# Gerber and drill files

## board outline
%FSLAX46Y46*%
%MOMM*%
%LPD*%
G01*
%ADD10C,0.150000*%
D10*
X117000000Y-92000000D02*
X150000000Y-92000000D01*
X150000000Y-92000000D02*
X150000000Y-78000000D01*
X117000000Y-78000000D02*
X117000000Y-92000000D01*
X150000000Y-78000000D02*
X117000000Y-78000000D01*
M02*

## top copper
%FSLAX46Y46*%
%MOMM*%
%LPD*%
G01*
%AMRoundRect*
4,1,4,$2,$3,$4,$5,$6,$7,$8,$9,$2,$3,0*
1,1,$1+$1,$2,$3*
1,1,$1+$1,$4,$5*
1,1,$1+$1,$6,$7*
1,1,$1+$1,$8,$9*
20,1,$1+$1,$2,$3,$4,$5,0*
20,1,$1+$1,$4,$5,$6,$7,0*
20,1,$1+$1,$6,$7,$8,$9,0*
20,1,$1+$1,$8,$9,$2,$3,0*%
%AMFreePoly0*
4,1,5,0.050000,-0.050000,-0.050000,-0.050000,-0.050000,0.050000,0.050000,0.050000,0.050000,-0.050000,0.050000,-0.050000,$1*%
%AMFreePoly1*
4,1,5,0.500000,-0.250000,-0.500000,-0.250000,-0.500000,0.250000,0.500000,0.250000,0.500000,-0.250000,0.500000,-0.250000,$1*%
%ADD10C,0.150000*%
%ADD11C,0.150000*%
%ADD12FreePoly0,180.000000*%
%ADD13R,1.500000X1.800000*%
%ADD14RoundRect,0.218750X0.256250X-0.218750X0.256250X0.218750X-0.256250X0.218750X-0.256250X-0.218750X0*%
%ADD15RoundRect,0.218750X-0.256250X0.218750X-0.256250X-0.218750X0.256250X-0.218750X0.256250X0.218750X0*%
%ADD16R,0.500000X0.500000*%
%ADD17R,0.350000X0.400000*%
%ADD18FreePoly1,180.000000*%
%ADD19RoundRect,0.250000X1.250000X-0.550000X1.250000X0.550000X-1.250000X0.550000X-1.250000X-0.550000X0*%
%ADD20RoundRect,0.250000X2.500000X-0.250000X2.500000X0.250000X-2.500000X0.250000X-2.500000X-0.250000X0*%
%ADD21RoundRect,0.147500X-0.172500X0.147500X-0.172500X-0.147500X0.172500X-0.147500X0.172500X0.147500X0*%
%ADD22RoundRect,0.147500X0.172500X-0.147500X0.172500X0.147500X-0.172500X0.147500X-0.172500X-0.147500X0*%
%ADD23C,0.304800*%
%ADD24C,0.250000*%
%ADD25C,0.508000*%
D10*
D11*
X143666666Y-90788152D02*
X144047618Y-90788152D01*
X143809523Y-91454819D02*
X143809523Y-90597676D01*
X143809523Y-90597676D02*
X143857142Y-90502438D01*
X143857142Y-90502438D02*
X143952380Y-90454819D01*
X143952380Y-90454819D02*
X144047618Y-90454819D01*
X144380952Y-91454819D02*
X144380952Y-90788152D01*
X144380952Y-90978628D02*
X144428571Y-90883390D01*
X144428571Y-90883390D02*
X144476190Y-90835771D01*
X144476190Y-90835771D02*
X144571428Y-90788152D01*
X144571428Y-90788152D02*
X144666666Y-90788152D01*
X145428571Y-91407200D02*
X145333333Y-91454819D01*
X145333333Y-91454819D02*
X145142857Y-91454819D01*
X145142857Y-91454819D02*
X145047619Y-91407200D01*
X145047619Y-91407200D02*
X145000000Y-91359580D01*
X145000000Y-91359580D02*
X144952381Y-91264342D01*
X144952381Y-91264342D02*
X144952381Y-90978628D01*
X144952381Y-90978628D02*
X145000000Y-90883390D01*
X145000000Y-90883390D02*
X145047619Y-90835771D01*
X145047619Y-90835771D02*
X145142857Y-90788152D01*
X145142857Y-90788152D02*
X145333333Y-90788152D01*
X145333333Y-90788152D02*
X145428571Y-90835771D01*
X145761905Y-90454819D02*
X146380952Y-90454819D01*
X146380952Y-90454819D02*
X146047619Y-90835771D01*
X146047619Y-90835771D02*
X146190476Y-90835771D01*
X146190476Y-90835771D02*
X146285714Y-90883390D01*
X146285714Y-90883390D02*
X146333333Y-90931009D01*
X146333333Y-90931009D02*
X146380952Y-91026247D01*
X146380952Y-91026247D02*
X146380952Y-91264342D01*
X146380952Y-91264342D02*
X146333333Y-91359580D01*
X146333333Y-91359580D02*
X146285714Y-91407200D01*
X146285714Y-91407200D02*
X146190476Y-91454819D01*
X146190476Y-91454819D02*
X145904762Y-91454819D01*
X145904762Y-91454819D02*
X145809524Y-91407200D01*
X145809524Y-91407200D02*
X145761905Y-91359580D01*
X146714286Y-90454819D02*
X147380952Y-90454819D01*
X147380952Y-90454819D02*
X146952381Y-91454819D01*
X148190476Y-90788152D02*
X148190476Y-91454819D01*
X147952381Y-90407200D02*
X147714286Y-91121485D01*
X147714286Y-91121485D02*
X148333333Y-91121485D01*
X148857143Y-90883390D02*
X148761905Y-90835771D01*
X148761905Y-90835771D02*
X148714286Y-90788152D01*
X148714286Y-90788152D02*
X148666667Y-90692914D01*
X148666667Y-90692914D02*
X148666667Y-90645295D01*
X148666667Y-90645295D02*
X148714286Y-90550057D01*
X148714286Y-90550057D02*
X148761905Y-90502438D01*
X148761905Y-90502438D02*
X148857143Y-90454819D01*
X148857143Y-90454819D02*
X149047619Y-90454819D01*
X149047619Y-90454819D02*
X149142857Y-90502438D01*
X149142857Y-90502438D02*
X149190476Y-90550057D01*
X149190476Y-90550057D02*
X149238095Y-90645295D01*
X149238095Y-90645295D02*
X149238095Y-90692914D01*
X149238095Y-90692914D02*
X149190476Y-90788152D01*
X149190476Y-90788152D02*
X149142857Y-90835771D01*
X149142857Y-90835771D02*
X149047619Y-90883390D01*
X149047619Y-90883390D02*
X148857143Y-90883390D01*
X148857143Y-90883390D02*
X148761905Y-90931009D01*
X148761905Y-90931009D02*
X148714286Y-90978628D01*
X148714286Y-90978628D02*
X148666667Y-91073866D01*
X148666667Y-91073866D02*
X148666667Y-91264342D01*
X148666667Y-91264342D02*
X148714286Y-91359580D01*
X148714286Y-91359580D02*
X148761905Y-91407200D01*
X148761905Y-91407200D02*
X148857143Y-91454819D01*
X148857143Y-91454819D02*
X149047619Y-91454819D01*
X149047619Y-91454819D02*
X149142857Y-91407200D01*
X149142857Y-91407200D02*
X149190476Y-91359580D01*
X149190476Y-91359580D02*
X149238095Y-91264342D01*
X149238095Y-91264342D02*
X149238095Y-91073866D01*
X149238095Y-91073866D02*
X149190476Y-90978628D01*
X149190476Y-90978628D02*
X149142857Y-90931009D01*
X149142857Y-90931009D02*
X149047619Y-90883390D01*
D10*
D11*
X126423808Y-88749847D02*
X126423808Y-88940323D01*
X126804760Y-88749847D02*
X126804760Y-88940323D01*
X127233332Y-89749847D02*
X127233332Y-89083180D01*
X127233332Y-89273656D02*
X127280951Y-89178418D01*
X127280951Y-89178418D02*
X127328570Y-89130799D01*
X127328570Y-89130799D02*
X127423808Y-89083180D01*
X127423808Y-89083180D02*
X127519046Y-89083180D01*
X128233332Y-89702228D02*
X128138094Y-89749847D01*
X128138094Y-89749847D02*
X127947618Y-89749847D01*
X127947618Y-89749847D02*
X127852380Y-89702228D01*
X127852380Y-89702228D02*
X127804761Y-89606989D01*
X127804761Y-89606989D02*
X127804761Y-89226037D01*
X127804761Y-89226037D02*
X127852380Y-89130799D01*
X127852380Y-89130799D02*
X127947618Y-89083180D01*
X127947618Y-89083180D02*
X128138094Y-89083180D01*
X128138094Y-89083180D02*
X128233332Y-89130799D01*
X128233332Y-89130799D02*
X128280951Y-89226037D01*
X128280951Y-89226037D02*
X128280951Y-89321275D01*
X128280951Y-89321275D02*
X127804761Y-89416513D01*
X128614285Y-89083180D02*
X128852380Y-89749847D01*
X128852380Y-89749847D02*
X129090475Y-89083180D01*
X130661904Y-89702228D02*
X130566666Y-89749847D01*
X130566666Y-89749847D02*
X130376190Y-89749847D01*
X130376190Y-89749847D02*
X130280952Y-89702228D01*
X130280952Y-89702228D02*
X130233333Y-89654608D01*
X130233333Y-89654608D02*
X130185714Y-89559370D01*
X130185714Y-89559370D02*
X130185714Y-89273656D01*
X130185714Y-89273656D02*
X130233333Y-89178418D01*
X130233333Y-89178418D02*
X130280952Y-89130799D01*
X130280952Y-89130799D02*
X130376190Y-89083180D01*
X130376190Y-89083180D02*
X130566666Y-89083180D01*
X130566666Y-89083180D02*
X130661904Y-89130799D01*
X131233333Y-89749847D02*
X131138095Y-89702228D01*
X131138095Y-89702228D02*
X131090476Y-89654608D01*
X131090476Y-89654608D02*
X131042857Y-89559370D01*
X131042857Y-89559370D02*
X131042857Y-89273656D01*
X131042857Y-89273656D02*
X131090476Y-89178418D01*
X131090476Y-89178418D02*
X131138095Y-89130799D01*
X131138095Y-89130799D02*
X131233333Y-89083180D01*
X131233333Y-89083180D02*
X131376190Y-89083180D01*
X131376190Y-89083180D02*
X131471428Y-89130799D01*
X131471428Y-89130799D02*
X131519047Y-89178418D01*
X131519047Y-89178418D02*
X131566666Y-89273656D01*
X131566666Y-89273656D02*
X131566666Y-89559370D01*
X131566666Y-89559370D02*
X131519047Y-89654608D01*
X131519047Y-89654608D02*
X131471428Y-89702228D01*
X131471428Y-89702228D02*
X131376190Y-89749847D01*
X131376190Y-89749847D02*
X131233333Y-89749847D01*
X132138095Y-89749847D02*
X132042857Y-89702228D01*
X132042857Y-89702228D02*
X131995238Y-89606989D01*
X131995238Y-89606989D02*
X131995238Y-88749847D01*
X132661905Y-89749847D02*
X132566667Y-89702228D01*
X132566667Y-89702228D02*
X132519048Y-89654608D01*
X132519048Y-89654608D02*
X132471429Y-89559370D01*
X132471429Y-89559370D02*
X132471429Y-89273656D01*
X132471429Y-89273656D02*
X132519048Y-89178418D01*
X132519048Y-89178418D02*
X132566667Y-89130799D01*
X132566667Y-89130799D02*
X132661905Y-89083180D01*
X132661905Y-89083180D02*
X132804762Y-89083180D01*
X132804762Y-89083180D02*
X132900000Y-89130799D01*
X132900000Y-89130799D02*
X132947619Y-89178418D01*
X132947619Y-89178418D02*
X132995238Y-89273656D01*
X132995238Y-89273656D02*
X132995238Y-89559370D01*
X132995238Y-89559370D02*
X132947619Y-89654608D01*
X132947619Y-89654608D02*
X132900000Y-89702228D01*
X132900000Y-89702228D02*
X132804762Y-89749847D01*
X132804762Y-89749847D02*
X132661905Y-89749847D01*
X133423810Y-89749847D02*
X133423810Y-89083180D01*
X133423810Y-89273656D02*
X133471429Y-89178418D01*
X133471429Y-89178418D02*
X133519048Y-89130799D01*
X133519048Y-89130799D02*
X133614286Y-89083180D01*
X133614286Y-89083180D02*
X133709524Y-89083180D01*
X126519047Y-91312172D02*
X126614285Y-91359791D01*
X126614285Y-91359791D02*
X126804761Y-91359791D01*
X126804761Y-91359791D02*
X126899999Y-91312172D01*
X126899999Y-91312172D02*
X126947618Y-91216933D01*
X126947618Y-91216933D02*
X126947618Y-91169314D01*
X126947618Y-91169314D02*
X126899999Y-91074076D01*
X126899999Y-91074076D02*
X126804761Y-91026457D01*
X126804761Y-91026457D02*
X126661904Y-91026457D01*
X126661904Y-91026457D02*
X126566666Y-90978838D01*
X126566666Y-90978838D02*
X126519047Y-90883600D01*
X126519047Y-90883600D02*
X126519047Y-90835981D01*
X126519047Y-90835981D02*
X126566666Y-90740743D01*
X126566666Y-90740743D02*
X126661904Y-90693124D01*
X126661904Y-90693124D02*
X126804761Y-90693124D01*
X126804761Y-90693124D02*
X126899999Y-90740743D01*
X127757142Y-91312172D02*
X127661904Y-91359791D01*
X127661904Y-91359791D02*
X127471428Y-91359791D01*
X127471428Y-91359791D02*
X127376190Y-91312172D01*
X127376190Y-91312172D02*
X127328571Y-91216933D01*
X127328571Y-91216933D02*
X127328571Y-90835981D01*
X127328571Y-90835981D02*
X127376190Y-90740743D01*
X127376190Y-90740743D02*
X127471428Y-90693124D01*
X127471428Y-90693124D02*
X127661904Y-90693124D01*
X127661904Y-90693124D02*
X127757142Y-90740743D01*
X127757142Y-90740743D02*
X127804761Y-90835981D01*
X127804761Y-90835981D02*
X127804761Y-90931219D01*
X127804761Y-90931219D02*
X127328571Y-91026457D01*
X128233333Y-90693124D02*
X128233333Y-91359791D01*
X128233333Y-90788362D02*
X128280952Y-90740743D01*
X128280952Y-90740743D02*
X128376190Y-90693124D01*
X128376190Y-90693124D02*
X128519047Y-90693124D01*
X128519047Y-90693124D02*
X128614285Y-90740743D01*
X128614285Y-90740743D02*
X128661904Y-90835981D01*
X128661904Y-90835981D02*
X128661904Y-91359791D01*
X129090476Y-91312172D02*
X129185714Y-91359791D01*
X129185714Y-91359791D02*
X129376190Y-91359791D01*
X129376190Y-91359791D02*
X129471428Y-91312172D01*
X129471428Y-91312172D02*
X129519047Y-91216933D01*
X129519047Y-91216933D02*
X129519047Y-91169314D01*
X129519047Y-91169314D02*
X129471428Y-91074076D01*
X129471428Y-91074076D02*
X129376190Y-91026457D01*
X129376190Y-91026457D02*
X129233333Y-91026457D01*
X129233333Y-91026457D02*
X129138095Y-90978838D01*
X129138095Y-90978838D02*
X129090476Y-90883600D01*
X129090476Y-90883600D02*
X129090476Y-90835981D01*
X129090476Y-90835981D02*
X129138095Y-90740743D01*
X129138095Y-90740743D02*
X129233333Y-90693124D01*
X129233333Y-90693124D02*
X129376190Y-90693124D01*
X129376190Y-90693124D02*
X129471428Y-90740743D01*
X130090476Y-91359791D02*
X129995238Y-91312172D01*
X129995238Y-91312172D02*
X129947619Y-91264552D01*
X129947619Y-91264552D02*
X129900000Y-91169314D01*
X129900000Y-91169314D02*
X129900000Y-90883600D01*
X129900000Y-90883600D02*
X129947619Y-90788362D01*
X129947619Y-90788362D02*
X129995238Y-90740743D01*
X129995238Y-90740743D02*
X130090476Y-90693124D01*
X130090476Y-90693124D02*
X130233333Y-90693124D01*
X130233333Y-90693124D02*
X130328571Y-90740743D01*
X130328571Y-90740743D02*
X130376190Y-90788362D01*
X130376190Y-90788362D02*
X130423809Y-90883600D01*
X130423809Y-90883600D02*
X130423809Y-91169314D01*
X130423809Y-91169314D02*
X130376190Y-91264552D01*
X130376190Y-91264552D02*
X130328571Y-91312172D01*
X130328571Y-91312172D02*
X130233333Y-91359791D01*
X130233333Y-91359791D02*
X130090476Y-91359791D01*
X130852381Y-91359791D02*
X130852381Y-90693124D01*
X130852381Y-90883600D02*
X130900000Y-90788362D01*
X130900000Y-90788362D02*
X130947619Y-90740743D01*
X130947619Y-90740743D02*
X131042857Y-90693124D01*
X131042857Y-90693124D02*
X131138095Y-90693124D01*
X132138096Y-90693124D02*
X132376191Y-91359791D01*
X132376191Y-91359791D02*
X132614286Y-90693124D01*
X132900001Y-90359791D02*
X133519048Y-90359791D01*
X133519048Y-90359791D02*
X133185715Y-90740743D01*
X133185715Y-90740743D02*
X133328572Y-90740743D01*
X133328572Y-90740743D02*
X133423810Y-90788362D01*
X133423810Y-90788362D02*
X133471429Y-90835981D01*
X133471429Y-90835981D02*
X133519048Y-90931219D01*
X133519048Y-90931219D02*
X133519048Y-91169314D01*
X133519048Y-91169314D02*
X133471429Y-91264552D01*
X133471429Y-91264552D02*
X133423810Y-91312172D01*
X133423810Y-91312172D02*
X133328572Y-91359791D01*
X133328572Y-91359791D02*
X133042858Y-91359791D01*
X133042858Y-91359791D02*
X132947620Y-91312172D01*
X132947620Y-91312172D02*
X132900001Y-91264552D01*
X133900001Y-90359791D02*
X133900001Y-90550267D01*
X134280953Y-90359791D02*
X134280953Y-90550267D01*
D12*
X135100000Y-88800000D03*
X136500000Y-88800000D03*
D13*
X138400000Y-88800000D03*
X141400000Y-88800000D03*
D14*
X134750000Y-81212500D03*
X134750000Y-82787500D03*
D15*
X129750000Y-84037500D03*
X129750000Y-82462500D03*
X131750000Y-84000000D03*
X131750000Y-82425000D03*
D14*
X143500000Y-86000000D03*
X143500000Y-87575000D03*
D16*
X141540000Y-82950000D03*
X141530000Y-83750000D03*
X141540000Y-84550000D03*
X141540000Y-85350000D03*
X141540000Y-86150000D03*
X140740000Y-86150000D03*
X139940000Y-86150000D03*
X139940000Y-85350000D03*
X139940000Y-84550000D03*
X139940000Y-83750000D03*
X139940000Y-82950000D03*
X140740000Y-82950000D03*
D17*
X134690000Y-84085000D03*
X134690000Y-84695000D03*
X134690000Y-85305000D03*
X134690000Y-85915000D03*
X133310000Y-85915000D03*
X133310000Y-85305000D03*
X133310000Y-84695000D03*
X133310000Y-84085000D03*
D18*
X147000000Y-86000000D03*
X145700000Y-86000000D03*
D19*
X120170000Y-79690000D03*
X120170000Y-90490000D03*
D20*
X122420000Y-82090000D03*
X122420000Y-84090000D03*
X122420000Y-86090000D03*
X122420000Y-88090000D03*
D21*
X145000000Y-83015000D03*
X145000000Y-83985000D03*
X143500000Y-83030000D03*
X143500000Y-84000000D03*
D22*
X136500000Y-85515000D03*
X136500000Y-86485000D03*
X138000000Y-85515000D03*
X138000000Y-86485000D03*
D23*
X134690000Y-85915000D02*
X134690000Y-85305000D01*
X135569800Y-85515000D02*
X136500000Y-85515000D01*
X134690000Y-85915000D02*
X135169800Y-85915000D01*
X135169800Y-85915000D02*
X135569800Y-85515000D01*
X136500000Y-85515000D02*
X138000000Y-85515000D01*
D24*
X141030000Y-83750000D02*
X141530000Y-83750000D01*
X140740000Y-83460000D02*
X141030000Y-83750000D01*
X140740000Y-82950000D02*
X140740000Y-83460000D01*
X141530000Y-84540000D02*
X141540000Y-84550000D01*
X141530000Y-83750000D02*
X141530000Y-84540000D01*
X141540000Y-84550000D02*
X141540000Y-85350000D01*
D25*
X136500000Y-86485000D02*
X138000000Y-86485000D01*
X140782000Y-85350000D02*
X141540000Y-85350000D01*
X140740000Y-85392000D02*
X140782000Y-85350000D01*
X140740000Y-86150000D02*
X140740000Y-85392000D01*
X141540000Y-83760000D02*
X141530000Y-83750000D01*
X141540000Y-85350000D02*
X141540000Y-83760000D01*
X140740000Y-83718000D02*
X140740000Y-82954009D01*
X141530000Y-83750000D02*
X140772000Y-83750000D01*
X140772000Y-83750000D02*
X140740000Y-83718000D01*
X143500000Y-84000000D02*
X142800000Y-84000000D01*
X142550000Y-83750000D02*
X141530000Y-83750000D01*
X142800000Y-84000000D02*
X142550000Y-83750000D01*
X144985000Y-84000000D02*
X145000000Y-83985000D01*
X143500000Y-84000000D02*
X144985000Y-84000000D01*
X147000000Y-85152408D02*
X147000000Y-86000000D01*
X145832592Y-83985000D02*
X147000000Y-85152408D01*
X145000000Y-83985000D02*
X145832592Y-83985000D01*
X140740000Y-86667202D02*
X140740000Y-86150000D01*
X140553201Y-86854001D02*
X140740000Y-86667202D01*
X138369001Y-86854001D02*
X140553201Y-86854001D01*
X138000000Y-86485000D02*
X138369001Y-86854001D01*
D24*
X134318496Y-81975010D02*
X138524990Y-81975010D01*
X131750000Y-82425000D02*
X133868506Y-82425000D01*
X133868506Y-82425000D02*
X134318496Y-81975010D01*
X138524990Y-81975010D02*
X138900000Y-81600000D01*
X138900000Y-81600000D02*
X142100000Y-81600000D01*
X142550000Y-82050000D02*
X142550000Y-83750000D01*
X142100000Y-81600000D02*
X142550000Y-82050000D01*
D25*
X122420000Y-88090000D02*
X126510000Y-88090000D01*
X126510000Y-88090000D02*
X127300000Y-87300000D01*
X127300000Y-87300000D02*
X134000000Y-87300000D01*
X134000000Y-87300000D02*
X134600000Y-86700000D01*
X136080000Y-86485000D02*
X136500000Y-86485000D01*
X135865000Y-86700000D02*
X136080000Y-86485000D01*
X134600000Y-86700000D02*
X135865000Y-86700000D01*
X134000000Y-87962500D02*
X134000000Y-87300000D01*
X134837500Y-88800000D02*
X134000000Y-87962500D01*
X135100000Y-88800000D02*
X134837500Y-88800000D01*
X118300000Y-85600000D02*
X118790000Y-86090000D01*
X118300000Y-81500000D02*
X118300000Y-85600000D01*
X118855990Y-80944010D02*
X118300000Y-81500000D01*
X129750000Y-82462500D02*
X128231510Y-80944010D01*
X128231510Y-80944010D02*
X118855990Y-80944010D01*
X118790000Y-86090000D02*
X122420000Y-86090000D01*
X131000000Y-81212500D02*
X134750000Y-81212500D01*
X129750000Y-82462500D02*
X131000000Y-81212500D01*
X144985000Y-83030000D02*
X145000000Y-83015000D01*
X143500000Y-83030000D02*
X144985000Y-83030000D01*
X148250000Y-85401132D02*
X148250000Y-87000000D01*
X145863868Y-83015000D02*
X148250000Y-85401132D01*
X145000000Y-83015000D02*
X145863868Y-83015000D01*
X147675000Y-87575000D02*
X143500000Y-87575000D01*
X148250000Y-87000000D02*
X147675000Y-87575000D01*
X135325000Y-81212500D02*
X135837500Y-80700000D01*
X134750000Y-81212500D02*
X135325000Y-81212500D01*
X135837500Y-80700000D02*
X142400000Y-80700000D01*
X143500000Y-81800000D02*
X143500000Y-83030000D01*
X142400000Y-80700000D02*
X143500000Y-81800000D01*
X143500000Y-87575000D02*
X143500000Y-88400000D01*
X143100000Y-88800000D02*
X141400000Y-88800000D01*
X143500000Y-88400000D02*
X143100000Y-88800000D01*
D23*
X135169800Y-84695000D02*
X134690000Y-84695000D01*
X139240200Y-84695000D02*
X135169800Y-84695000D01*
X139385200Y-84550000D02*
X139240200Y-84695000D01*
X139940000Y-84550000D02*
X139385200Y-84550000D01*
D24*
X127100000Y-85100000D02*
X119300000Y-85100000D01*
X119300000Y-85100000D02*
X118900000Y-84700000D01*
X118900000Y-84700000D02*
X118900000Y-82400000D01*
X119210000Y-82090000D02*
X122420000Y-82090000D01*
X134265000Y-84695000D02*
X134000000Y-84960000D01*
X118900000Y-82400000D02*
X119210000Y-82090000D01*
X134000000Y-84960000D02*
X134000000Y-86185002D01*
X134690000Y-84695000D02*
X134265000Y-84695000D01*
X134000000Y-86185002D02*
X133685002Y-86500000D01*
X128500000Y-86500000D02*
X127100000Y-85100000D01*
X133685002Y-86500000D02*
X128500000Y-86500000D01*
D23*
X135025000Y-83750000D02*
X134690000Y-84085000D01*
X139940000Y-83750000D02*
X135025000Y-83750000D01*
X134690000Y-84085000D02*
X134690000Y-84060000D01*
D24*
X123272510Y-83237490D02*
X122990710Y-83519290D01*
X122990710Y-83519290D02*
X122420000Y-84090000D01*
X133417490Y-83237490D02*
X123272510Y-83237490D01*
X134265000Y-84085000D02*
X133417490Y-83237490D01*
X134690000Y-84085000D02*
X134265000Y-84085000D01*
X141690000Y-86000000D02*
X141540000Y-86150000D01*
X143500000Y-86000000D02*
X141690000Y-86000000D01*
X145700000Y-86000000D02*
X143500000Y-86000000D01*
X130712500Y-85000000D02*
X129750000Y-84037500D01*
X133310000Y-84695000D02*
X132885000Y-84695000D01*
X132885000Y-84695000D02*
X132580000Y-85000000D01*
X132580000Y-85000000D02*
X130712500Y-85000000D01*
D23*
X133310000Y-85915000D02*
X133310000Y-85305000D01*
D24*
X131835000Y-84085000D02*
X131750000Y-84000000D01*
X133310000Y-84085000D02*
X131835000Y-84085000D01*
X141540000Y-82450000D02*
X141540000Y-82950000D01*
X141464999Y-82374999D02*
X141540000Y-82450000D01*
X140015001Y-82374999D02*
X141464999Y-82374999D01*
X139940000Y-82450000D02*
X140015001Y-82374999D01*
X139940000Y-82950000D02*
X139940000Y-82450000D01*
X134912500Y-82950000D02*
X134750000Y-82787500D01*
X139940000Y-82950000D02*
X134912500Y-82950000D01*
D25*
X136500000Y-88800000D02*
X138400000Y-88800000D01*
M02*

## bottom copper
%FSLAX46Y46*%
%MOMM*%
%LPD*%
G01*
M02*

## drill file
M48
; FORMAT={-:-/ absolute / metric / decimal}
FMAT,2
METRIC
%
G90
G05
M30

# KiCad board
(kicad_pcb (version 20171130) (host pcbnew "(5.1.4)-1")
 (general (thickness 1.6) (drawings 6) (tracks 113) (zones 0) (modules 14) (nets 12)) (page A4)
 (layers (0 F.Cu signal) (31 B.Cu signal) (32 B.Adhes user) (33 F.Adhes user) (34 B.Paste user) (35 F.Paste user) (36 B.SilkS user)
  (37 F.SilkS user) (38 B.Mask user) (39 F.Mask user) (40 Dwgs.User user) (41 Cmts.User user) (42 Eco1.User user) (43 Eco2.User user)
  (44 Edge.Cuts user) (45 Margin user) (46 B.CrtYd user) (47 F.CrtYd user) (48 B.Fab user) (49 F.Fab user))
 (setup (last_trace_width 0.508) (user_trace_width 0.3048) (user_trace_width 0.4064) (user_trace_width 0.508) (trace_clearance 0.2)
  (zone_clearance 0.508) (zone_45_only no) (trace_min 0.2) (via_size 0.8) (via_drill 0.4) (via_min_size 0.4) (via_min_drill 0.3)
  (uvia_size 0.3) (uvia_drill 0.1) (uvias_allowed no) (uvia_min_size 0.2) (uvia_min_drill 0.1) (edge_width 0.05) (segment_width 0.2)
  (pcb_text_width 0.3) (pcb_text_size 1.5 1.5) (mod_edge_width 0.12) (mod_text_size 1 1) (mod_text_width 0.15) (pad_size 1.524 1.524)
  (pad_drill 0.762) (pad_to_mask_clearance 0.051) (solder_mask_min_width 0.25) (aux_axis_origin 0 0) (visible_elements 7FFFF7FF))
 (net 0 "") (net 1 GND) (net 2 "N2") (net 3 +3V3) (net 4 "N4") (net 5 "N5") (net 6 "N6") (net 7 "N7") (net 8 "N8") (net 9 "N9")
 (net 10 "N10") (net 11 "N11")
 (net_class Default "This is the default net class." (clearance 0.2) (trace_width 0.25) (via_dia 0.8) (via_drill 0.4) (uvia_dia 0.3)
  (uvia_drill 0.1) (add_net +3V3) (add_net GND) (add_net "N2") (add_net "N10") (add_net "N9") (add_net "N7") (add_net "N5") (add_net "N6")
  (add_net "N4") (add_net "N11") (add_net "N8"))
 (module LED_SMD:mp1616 (layer F.Cu) (at 135.8 88.9 180)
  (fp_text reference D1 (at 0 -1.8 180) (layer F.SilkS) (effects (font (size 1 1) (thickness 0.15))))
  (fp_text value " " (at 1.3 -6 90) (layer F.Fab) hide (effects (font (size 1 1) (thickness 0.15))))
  (pad 1 smd custom (at 0.7 0.1 180) (size 0.1 0.1) (layers F.Cu F.Paste F.Mask) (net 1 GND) (options (clearance outline) (anchor rect))
   (primitives))
  (pad 2 smd custom (at -0.7 0.1 180) (size 0.1 0.1) (layers F.Cu F.Paste F.Mask) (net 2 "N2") (options (clearance outline) (anchor rect))
   (primitives)))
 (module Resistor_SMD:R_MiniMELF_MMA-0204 (layer F.Cu) (at 139.9 88.8 180)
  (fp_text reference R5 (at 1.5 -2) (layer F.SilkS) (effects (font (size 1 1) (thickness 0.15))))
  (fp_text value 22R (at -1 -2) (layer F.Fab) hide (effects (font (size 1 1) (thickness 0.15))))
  (pad 2 smd rect (at 1.5 0 180) (size 1.5 1.8) (layers F.Cu F.Paste F.Mask) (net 2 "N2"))
  (pad 1 smd rect (at -1.5 0 180) (size 1.5 1.8) (layers F.Cu F.Paste F.Mask) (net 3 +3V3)))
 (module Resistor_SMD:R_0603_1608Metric (layer F.Cu) (at 134.75 82 90)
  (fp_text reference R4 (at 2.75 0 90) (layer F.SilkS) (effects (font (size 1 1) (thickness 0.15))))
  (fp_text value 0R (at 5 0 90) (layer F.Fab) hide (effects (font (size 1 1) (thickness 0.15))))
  (pad 2 smd roundrect (at 0.7875 0 90) (size 0.875 0.95) (layers F.Cu F.Paste F.Mask) (roundrect_rratio 0.25) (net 3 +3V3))
  (pad 1 smd roundrect (at -0.7875 0 90) (size 0.875 0.95) (layers F.Cu F.Paste F.Mask) (roundrect_rratio 0.25) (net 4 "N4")))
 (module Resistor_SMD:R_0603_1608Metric (layer F.Cu) (at 129.75 83.25 270)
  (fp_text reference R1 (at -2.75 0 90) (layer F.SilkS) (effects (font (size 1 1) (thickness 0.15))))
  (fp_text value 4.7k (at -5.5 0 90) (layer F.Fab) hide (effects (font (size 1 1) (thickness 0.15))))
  (pad 2 smd roundrect (at 0.7875 0 270) (size 0.875 0.95) (layers F.Cu F.Paste F.Mask) (roundrect_rratio 0.25) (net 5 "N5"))
  (pad 1 smd roundrect (at -0.7875 0 270) (size 0.875 0.95) (layers F.Cu F.Paste F.Mask) (roundrect_rratio 0.25) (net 3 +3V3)))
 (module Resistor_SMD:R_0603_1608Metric (layer F.Cu) (at 131.75 83.2125 270)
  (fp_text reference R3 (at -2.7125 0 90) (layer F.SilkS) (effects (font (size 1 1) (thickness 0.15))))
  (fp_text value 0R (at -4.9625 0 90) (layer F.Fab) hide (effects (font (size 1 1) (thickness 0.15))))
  (pad 2 smd roundrect (at 0.7875 0 270) (size 0.875 0.95) (layers F.Cu F.Paste F.Mask) (roundrect_rratio 0.25) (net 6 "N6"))
  (pad 1 smd roundrect (at -0.7875 0 270) (size 0.875 0.95) (layers F.Cu F.Paste F.Mask) (roundrect_rratio 0.25) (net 1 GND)))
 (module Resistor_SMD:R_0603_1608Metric (layer F.Cu) (at 143.5 86.7875 90)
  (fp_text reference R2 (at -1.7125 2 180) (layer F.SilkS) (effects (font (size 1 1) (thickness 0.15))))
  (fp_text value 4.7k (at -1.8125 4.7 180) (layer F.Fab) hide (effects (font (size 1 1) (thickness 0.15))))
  (pad 2 smd roundrect (at 0.7875 0 90) (size 0.875 0.95) (layers F.Cu F.Paste F.Mask) (roundrect_rratio 0.25) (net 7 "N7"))
  (pad 1 smd roundrect (at -0.7875 0 90) (size 0.875 0.95) (layers F.Cu F.Paste F.Mask) (roundrect_rratio 0.25) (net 3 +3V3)))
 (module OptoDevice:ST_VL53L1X (layer F.Cu) (at 140.74 84.55 270)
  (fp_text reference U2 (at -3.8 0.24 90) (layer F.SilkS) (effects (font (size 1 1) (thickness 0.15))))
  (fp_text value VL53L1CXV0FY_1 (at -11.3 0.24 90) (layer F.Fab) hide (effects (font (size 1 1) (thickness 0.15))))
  (pad 1 smd rect (at -1.6 -0.8) (size 0.5 0.5) (layers F.Cu F.Paste F.Mask) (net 4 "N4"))
  (pad 2 smd rect (at -0.8 -0.79) (size 0.5 0.5) (layers F.Cu F.Paste F.Mask) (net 1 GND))
  (pad 3 smd rect (at 0 -0.8) (size 0.5 0.5) (layers F.Cu F.Paste F.Mask) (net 1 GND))
  (pad 4 smd rect (at 0.8 -0.8) (size 0.5 0.5) (layers F.Cu F.Paste F.Mask) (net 1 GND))
  (pad 5 smd rect (at 1.6 -0.8) (size 0.5 0.5) (layers F.Cu F.Paste F.Mask) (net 7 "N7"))
  (pad 6 smd rect (at 1.6 0) (size 0.5 0.5) (layers F.Cu F.Paste F.Mask) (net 1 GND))
  (pad 7 smd rect (at 1.6 0.8) (size 0.5 0.5) (layers F.Cu F.Paste F.Mask) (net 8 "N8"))
  (pad 8 smd rect (at 0.8 0.8) (size 0.5 0.5) (layers F.Cu F.Paste F.Mask))
  (pad 9 smd rect (at 0 0.8) (size 0.5 0.5) (layers F.Cu F.Paste F.Mask) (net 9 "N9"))
  (pad 10 smd rect (at -0.8 0.8) (size 0.5 0.5) (layers F.Cu F.Paste F.Mask) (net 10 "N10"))
  (pad 11 smd rect (at -1.6 0.8) (size 0.5 0.5) (layers F.Cu F.Paste F.Mask) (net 4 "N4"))
  (pad 12 smd rect (at -1.6 0) (size 0.5 0.5) (layers F.Cu F.Paste F.Mask) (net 1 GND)))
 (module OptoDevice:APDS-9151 (layer F.Cu) (at 134 85)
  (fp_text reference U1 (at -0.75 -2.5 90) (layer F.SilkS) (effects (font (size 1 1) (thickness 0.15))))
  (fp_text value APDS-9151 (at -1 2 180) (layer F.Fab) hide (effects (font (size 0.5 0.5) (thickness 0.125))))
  (pad 8 smd rect (at 0.69 -0.915) (size 0.35 0.4) (layers F.Cu F.Paste F.Mask) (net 10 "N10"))
  (pad 7 smd rect (at 0.69 -0.305) (size 0.35 0.4) (layers F.Cu F.Paste F.Mask) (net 9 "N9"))
  (pad 6 smd rect (at 0.69 0.305 180) (size 0.35 0.4) (layers F.Cu F.Paste F.Mask) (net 3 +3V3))
  (pad 5 smd rect (at 0.69 0.915) (size 0.35 0.4) (layers F.Cu F.Paste F.Mask) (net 3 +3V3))
  (pad 4 smd rect (at -0.69 0.915) (size 0.35 0.4) (layers F.Cu F.Paste F.Mask) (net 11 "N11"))
  (pad 3 smd rect (at -0.69 0.305) (size 0.35 0.4) (layers F.Cu F.Paste F.Mask) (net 11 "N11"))
  (pad 2 smd rect (at -0.69 -0.305) (size 0.35 0.4) (layers F.Cu F.Paste F.Mask) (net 5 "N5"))
  (pad 1 smd rect (at -0.69 -0.915) (size 0.35 0.4) (layers F.Cu F.Paste F.Mask) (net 6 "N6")))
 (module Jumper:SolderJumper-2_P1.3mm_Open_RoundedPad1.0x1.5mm (layer F.Cu) (at 146.35 86 180)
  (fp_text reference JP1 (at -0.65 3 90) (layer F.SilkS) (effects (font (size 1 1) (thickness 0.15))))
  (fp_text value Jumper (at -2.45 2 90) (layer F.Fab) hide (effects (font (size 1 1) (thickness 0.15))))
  (pad 1 smd custom (at -0.65 0 180) (size 1 0.5) (layers F.Cu F.Mask) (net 1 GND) (zone_connect 2)
   (options (clearance outline) (anchor rect)) (primitives))
  (pad 2 smd custom (at 0.65 0 180) (size 1 0.5) (layers F.Cu F.Mask) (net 7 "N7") (zone_connect 2)
   (options (clearance outline) (anchor rect)) (primitives)))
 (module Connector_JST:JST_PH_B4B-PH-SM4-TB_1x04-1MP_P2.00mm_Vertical (layer F.Cu) (at 121.92 85.09 90)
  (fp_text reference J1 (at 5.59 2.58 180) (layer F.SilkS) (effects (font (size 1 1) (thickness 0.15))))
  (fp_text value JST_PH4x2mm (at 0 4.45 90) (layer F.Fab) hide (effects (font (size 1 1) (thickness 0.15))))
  (pad MP smd roundrect (at 5.4 -1.75 90) (size 1.6 3) (layers F.Cu F.Paste F.Mask) (roundrect_rratio 0.15625))
  (pad MP smd roundrect (at -5.4 -1.75 90) (size 1.6 3) (layers F.Cu F.Paste F.Mask) (roundrect_rratio 0.15625))
  (pad 4 smd roundrect (at 3 0.5 90) (size 1 5.5) (layers F.Cu F.Paste F.Mask) (roundrect_rratio 0.25) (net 9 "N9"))
  (pad 3 smd roundrect (at 1 0.5 90) (size 1 5.5) (layers F.Cu F.Paste F.Mask) (roundrect_rratio 0.25) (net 10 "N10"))
  (pad 2 smd roundrect (at -1 0.5 90) (size 1 5.5) (layers F.Cu F.Paste F.Mask) (roundrect_rratio 0.25) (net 3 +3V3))
  (pad 1 smd roundrect (at -3 0.5 90) (size 1 5.5) (layers F.Cu F.Paste F.Mask) (roundrect_rratio 0.25) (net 1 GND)))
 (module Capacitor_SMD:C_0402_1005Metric (layer F.Cu) (at 145 83.5 270)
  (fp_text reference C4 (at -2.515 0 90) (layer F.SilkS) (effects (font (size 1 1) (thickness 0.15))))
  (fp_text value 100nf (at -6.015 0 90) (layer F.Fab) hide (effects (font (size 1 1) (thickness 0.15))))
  (pad 1 smd roundrect (at -0.485 0 270) (size 0.59 0.64) (layers F.Cu F.Paste F.Mask) (roundrect_rratio 0.25) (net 3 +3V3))
  (pad 2 smd roundrect (at 0.485 0 270) (size 0.59 0.64) (layers F.Cu F.Paste F.Mask) (roundrect_rratio 0.25) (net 1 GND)))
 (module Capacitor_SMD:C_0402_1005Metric (layer F.Cu) (at 143.5 83.515 270)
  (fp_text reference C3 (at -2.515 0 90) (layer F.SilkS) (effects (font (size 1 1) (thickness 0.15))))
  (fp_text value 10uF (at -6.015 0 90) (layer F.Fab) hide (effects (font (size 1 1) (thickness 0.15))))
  (pad 1 smd roundrect (at -0.485 0 270) (size 0.59 0.64) (layers F.Cu F.Paste F.Mask) (roundrect_rratio 0.25) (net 3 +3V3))
  (pad 2 smd roundrect (at 0.485 0 270) (size 0.59 0.64) (layers F.Cu F.Paste F.Mask) (roundrect_rratio 0.25) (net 1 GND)))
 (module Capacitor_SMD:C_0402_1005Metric (layer F.Cu) (at 136.5 86 90)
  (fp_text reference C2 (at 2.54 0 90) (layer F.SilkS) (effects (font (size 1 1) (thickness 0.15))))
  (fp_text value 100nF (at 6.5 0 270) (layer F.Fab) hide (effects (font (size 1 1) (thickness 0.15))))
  (pad 2 smd roundrect (at 0.485 0 90) (size 0.59 0.64) (layers F.Cu F.Paste F.Mask) (roundrect_rratio 0.25) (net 3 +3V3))
  (pad 1 smd roundrect (at -0.485 0 90) (size 0.59 0.64) (layers F.Cu F.Paste F.Mask) (roundrect_rratio 0.25) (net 1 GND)))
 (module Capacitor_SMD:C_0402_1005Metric (layer F.Cu) (at 138 86 90)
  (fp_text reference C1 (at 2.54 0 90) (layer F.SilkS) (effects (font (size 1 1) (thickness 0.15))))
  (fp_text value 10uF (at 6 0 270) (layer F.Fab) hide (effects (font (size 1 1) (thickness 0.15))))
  (pad 2 smd roundrect (at 0.485 0 90) (size 0.59 0.64) (layers F.Cu F.Paste F.Mask) (roundrect_rratio 0.25) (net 3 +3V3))
  (pad 1 smd roundrect (at -0.485 0 90) (size 0.59 0.64) (layers F.Cu F.Paste F.Mask) (roundrect_rratio 0.25) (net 1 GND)))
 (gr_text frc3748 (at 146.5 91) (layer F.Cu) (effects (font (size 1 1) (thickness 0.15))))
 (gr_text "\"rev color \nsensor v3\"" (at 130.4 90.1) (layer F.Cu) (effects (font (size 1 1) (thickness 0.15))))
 (gr_line (start 117 92) (end 150 92) (layer Edge.Cuts) (width 0.15))
 (gr_line (start 150 92) (end 150 78) (layer Edge.Cuts) (width 0.15))
 (gr_line (start 117 78) (end 117 92) (layer Edge.Cuts) (width 0.15))
 (gr_line (start 150 78) (end 117 78) (layer Edge.Cuts) (width 0.15))
 (segment (start 134.69 85.915) (end 134.69 85.305) (width 0.3048) (layer F.Cu) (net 3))
 (segment (start 135.5698 85.515) (end 136.5 85.515) (width 0.3048) (layer F.Cu) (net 3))
 (segment (start 134.69 85.915) (end 135.1698 85.915) (width 0.3048) (layer F.Cu) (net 3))
 (segment (start 135.1698 85.915) (end 135.5698 85.515) (width 0.3048) (layer F.Cu) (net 3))
 (segment (start 136.5 85.515) (end 138 85.515) (width 0.3048) (layer F.Cu) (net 3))
 (segment (start 141.03 83.75) (end 141.53 83.75) (width 0.25) (layer F.Cu) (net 1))
 (segment (start 140.74 83.46) (end 141.03 83.75) (width 0.25) (layer F.Cu) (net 1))
 (segment (start 140.74 82.95) (end 140.74 83.46) (width 0.25) (layer F.Cu) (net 1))
 (segment (start 141.53 84.54) (end 141.54 84.55) (width 0.25) (layer F.Cu) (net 1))
 (segment (start 141.53 83.75) (end 141.53 84.54) (width 0.25) (layer F.Cu) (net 1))
 (segment (start 141.54 84.55) (end 141.54 85.35) (width 0.25) (layer F.Cu) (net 1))
 (segment (start 136.5 86.485) (end 138 86.485) (width 0.508) (layer F.Cu) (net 1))
 (segment (start 140.782 85.35) (end 141.54 85.35) (width 0.508) (layer F.Cu) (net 1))
 (segment (start 140.74 85.392) (end 140.782 85.35) (width 0.508) (layer F.Cu) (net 1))
 (segment (start 140.74 86.15) (end 140.74 85.392) (width 0.508) (layer F.Cu) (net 1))
 (segment (start 141.54 83.76) (end 141.53 83.75) (width 0.508) (layer F.Cu) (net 1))
 (segment (start 141.54 85.35) (end 141.54 83.76) (width 0.508) (layer F.Cu) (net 1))
 (segment (start 140.74 83.718) (end 140.74 82.954009) (width 0.508) (layer F.Cu) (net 1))
 (segment (start 141.53 83.75) (end 140.772 83.75) (width 0.508) (layer F.Cu) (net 1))
 (segment (start 140.772 83.75) (end 140.74 83.718) (width 0.508) (layer F.Cu) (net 1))
 (segment (start 143.5 84) (end 142.8 84) (width 0.508) (layer F.Cu) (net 1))
 (segment (start 142.55 83.75) (end 141.53 83.75) (width 0.508) (layer F.Cu) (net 1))
 (segment (start 142.8 84) (end 142.55 83.75) (width 0.508) (layer F.Cu) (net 1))
 (segment (start 144.985 84) (end 145 83.985) (width 0.508) (layer F.Cu) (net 1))
 (segment (start 143.5 84) (end 144.985 84) (width 0.508) (layer F.Cu) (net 1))
 (segment (start 147 85.152408) (end 147 86) (width 0.508) (layer F.Cu) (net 1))
 (segment (start 145.832592 83.985) (end 147 85.152408) (width 0.508) (layer F.Cu) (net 1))
 (segment (start 145 83.985) (end 145.832592 83.985) (width 0.508) (layer F.Cu) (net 1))
 (segment (start 140.74 86.667202) (end 140.74 86.15) (width 0.508) (layer F.Cu) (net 1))
 (segment (start 140.553201 86.854001) (end 140.74 86.667202) (width 0.508) (layer F.Cu) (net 1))
 (segment (start 138.369001 86.854001) (end 140.553201 86.854001) (width 0.508) (layer F.Cu) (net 1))
 (segment (start 138 86.485) (end 138.369001 86.854001) (width 0.508) (layer F.Cu) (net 1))
 (segment (start 134.318496 81.97501) (end 138.52499 81.97501) (width 0.25) (layer F.Cu) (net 1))
 (segment (start 131.75 82.425) (end 133.868506 82.425) (width 0.25) (layer F.Cu) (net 1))
 (segment (start 133.868506 82.425) (end 134.318496 81.97501) (width 0.25) (layer F.Cu) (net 1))
 (segment (start 138.52499 81.97501) (end 138.9 81.6) (width 0.25) (layer F.Cu) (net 1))
 (segment (start 138.9 81.6) (end 142.1 81.6) (width 0.25) (layer F.Cu) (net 1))
 (segment (start 142.55 82.05) (end 142.55 83.75) (width 0.25) (layer F.Cu) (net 1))
 (segment (start 142.1 81.6) (end 142.55 82.05) (width 0.25) (layer F.Cu) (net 1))
 (segment (start 122.42 88.09) (end 126.51 88.09) (width 0.508) (layer F.Cu) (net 1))
 (segment (start 126.51 88.09) (end 127.3 87.3) (width 0.508) (layer F.Cu) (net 1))
 (segment (start 127.3 87.3) (end 134 87.3) (width 0.508) (layer F.Cu) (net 1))
 (segment (start 134 87.3) (end 134.6 86.7) (width 0.508) (layer F.Cu) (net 1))
 (segment (start 136.08 86.485) (end 136.5 86.485) (width 0.508) (layer F.Cu) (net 1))
 (segment (start 135.865 86.7) (end 136.08 86.485) (width 0.508) (layer F.Cu) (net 1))
 (segment (start 134.6 86.7) (end 135.865 86.7) (width 0.508) (layer F.Cu) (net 1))
 (segment (start 134 87.9625) (end 134 87.3) (width 0.508) (layer F.Cu) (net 1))
 (segment (start 134.8375 88.8) (end 134 87.9625) (width 0.508) (layer F.Cu) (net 1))
 (segment (start 135.1 88.8) (end 134.8375 88.8) (width 0.508) (layer F.Cu) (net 1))
 (segment (start 118.3 85.6) (end 118.79 86.09) (width 0.508) (layer F.Cu) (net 3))
 (segment (start 118.3 81.5) (end 118.3 85.6) (width 0.508) (layer F.Cu) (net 3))
 (segment (start 118.85599 80.94401) (end 118.3 81.5) (width 0.508) (layer F.Cu) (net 3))
 (segment (start 129.75 82.4625) (end 128.23151 80.94401) (width 0.508) (layer F.Cu) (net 3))
 (segment (start 128.23151 80.94401) (end 118.85599 80.94401) (width 0.508) (layer F.Cu) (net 3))
 (segment (start 118.79 86.09) (end 122.42 86.09) (width 0.508) (layer F.Cu) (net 3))
 (segment (start 131 81.2125) (end 134.75 81.2125) (width 0.508) (layer F.Cu) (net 3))
 (segment (start 129.75 82.4625) (end 131 81.2125) (width 0.508) (layer F.Cu) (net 3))
 (segment (start 144.985 83.03) (end 145 83.015) (width 0.508) (layer F.Cu) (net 3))
 (segment (start 143.5 83.03) (end 144.985 83.03) (width 0.508) (layer F.Cu) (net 3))
 (segment (start 148.25 85.401132) (end 148.25 87) (width 0.508) (layer F.Cu) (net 3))
 (segment (start 145.863868 83.015) (end 148.25 85.401132) (width 0.508) (layer F.Cu) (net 3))
 (segment (start 145 83.015) (end 145.863868 83.015) (width 0.508) (layer F.Cu) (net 3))
 (segment (start 147.675 87.575) (end 143.5 87.575) (width 0.508) (layer F.Cu) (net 3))
 (segment (start 148.25 87) (end 147.675 87.575) (width 0.508) (layer F.Cu) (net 3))
 (segment (start 135.325 81.2125) (end 135.8375 80.7) (width 0.508) (layer F.Cu) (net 3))
 (segment (start 134.75 81.2125) (end 135.325 81.2125) (width 0.508) (layer F.Cu) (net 3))
 (segment (start 135.8375 80.7) (end 142.4 80.7) (width 0.508) (layer F.Cu) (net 3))
 (segment (start 143.5 81.8) (end 143.5 83.03) (width 0.508) (layer F.Cu) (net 3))
 (segment (start 142.4 80.7) (end 143.5 81.8) (width 0.508) (layer F.Cu) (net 3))
 (segment (start 143.5 87.575) (end 143.5 88.4) (width 0.508) (layer F.Cu) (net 3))
 (segment (start 143.1 88.8) (end 141.4 88.8) (width 0.508) (layer F.Cu) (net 3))
 (segment (start 143.5 88.4) (end 143.1 88.8) (width 0.508) (layer F.Cu) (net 3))
 (segment (start 135.1698 84.695) (end 134.69 84.695) (width 0.3048) (layer F.Cu) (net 9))
 (segment (start 139.2402 84.695) (end 135.1698 84.695) (width 0.3048) (layer F.Cu) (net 9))
 (segment (start 139.3852 84.55) (end 139.2402 84.695) (width 0.3048) (layer F.Cu) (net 9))
 (segment (start 139.94 84.55) (end 139.3852 84.55) (width 0.3048) (layer F.Cu) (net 9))
 (segment (start 127.1 85.1) (end 119.3 85.1) (width 0.25) (layer F.Cu) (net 9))
 (segment (start 119.3 85.1) (end 118.9 84.7) (width 0.25) (layer F.Cu) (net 9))
 (segment (start 118.9 84.7) (end 118.9 82.4) (width 0.25) (layer F.Cu) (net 9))
 (segment (start 119.21 82.09) (end 122.42 82.09) (width 0.25) (layer F.Cu) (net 9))
 (segment (start 134.265 84.695) (end 134 84.96) (width 0.25) (layer F.Cu) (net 9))
 (segment (start 118.9 82.4) (end 119.21 82.09) (width 0.25) (layer F.Cu) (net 9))
 (segment (start 134 84.96) (end 134 86.185002) (width 0.25) (layer F.Cu) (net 9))
 (segment (start 134.69 84.695) (end 134.265 84.695) (width 0.25) (layer F.Cu) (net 9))
 (segment (start 134 86.185002) (end 133.685002 86.5) (width 0.25) (layer F.Cu) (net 9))
 (segment (start 128.5 86.5) (end 127.1 85.1) (width 0.25) (layer F.Cu) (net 9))
 (segment (start 133.685002 86.5) (end 128.5 86.5) (width 0.25) (layer F.Cu) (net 9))
 (segment (start 135.025 83.75) (end 134.69 84.085) (width 0.3048) (layer F.Cu) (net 10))
 (segment (start 139.94 83.75) (end 135.025 83.75) (width 0.3048) (layer F.Cu) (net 10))
 (segment (start 134.69 84.085) (end 134.69 84.06) (width 0.3048) (layer F.Cu) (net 10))
 (segment (start 123.27251 83.23749) (end 122.99071 83.51929) (width 0.25) (layer F.Cu) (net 10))
 (segment (start 122.99071 83.51929) (end 122.42 84.09) (width 0.25) (layer F.Cu) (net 10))
 (segment (start 133.41749 83.23749) (end 123.27251 83.23749) (width 0.25) (layer F.Cu) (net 10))
 (segment (start 134.265 84.085) (end 133.41749 83.23749) (width 0.25) (layer F.Cu) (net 10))
 (segment (start 134.69 84.085) (end 134.265 84.085) (width 0.25) (layer F.Cu) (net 10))
 (segment (start 141.69 86) (end 141.54 86.15) (width 0.25) (layer F.Cu) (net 7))
 (segment (start 143.5 86) (end 141.69 86) (width 0.25) (layer F.Cu) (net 7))
 (segment (start 145.7 86) (end 143.5 86) (width 0.25) (layer F.Cu) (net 7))
 (segment (start 130.7125 85) (end 129.75 84.0375) (width 0.25) (layer F.Cu) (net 5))
 (segment (start 133.31 84.695) (end 132.885 84.695) (width 0.25) (layer F.Cu) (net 5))
 (segment (start 132.885 84.695) (end 132.58 85) (width 0.25) (layer F.Cu) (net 5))
 (segment (start 132.58 85) (end 130.7125 85) (width 0.25) (layer F.Cu) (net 5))
 (segment (start 133.31 85.915) (end 133.31 85.305) (width 0.3048) (layer F.Cu) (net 11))
 (segment (start 131.835 84.085) (end 131.75 84) (width 0.25) (layer F.Cu) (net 6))
 (segment (start 133.31 84.085) (end 131.835 84.085) (width 0.25) (layer F.Cu) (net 6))
 (segment (start 141.54 82.45) (end 141.54 82.95) (width 0.25) (layer F.Cu) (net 4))
 (segment (start 141.464999 82.374999) (end 141.54 82.45) (width 0.25) (layer F.Cu) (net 4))
 (segment (start 140.015001 82.374999) (end 141.464999 82.374999) (width 0.25) (layer F.Cu) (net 4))
 (segment (start 139.94 82.45) (end 140.015001 82.374999) (width 0.25) (layer F.Cu) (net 4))
 (segment (start 139.94 82.95) (end 139.94 82.45) (width 0.25) (layer F.Cu) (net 4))
 (segment (start 134.9125 82.95) (end 134.75 82.7875) (width 0.25) (layer F.Cu) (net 4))
 (segment (start 139.94 82.95) (end 134.9125 82.95) (width 0.25) (layer F.Cu) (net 4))
 (segment (start 136.5 88.8) (end 138.4 88.8) (width 0.508) (layer F.Cu) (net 2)))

